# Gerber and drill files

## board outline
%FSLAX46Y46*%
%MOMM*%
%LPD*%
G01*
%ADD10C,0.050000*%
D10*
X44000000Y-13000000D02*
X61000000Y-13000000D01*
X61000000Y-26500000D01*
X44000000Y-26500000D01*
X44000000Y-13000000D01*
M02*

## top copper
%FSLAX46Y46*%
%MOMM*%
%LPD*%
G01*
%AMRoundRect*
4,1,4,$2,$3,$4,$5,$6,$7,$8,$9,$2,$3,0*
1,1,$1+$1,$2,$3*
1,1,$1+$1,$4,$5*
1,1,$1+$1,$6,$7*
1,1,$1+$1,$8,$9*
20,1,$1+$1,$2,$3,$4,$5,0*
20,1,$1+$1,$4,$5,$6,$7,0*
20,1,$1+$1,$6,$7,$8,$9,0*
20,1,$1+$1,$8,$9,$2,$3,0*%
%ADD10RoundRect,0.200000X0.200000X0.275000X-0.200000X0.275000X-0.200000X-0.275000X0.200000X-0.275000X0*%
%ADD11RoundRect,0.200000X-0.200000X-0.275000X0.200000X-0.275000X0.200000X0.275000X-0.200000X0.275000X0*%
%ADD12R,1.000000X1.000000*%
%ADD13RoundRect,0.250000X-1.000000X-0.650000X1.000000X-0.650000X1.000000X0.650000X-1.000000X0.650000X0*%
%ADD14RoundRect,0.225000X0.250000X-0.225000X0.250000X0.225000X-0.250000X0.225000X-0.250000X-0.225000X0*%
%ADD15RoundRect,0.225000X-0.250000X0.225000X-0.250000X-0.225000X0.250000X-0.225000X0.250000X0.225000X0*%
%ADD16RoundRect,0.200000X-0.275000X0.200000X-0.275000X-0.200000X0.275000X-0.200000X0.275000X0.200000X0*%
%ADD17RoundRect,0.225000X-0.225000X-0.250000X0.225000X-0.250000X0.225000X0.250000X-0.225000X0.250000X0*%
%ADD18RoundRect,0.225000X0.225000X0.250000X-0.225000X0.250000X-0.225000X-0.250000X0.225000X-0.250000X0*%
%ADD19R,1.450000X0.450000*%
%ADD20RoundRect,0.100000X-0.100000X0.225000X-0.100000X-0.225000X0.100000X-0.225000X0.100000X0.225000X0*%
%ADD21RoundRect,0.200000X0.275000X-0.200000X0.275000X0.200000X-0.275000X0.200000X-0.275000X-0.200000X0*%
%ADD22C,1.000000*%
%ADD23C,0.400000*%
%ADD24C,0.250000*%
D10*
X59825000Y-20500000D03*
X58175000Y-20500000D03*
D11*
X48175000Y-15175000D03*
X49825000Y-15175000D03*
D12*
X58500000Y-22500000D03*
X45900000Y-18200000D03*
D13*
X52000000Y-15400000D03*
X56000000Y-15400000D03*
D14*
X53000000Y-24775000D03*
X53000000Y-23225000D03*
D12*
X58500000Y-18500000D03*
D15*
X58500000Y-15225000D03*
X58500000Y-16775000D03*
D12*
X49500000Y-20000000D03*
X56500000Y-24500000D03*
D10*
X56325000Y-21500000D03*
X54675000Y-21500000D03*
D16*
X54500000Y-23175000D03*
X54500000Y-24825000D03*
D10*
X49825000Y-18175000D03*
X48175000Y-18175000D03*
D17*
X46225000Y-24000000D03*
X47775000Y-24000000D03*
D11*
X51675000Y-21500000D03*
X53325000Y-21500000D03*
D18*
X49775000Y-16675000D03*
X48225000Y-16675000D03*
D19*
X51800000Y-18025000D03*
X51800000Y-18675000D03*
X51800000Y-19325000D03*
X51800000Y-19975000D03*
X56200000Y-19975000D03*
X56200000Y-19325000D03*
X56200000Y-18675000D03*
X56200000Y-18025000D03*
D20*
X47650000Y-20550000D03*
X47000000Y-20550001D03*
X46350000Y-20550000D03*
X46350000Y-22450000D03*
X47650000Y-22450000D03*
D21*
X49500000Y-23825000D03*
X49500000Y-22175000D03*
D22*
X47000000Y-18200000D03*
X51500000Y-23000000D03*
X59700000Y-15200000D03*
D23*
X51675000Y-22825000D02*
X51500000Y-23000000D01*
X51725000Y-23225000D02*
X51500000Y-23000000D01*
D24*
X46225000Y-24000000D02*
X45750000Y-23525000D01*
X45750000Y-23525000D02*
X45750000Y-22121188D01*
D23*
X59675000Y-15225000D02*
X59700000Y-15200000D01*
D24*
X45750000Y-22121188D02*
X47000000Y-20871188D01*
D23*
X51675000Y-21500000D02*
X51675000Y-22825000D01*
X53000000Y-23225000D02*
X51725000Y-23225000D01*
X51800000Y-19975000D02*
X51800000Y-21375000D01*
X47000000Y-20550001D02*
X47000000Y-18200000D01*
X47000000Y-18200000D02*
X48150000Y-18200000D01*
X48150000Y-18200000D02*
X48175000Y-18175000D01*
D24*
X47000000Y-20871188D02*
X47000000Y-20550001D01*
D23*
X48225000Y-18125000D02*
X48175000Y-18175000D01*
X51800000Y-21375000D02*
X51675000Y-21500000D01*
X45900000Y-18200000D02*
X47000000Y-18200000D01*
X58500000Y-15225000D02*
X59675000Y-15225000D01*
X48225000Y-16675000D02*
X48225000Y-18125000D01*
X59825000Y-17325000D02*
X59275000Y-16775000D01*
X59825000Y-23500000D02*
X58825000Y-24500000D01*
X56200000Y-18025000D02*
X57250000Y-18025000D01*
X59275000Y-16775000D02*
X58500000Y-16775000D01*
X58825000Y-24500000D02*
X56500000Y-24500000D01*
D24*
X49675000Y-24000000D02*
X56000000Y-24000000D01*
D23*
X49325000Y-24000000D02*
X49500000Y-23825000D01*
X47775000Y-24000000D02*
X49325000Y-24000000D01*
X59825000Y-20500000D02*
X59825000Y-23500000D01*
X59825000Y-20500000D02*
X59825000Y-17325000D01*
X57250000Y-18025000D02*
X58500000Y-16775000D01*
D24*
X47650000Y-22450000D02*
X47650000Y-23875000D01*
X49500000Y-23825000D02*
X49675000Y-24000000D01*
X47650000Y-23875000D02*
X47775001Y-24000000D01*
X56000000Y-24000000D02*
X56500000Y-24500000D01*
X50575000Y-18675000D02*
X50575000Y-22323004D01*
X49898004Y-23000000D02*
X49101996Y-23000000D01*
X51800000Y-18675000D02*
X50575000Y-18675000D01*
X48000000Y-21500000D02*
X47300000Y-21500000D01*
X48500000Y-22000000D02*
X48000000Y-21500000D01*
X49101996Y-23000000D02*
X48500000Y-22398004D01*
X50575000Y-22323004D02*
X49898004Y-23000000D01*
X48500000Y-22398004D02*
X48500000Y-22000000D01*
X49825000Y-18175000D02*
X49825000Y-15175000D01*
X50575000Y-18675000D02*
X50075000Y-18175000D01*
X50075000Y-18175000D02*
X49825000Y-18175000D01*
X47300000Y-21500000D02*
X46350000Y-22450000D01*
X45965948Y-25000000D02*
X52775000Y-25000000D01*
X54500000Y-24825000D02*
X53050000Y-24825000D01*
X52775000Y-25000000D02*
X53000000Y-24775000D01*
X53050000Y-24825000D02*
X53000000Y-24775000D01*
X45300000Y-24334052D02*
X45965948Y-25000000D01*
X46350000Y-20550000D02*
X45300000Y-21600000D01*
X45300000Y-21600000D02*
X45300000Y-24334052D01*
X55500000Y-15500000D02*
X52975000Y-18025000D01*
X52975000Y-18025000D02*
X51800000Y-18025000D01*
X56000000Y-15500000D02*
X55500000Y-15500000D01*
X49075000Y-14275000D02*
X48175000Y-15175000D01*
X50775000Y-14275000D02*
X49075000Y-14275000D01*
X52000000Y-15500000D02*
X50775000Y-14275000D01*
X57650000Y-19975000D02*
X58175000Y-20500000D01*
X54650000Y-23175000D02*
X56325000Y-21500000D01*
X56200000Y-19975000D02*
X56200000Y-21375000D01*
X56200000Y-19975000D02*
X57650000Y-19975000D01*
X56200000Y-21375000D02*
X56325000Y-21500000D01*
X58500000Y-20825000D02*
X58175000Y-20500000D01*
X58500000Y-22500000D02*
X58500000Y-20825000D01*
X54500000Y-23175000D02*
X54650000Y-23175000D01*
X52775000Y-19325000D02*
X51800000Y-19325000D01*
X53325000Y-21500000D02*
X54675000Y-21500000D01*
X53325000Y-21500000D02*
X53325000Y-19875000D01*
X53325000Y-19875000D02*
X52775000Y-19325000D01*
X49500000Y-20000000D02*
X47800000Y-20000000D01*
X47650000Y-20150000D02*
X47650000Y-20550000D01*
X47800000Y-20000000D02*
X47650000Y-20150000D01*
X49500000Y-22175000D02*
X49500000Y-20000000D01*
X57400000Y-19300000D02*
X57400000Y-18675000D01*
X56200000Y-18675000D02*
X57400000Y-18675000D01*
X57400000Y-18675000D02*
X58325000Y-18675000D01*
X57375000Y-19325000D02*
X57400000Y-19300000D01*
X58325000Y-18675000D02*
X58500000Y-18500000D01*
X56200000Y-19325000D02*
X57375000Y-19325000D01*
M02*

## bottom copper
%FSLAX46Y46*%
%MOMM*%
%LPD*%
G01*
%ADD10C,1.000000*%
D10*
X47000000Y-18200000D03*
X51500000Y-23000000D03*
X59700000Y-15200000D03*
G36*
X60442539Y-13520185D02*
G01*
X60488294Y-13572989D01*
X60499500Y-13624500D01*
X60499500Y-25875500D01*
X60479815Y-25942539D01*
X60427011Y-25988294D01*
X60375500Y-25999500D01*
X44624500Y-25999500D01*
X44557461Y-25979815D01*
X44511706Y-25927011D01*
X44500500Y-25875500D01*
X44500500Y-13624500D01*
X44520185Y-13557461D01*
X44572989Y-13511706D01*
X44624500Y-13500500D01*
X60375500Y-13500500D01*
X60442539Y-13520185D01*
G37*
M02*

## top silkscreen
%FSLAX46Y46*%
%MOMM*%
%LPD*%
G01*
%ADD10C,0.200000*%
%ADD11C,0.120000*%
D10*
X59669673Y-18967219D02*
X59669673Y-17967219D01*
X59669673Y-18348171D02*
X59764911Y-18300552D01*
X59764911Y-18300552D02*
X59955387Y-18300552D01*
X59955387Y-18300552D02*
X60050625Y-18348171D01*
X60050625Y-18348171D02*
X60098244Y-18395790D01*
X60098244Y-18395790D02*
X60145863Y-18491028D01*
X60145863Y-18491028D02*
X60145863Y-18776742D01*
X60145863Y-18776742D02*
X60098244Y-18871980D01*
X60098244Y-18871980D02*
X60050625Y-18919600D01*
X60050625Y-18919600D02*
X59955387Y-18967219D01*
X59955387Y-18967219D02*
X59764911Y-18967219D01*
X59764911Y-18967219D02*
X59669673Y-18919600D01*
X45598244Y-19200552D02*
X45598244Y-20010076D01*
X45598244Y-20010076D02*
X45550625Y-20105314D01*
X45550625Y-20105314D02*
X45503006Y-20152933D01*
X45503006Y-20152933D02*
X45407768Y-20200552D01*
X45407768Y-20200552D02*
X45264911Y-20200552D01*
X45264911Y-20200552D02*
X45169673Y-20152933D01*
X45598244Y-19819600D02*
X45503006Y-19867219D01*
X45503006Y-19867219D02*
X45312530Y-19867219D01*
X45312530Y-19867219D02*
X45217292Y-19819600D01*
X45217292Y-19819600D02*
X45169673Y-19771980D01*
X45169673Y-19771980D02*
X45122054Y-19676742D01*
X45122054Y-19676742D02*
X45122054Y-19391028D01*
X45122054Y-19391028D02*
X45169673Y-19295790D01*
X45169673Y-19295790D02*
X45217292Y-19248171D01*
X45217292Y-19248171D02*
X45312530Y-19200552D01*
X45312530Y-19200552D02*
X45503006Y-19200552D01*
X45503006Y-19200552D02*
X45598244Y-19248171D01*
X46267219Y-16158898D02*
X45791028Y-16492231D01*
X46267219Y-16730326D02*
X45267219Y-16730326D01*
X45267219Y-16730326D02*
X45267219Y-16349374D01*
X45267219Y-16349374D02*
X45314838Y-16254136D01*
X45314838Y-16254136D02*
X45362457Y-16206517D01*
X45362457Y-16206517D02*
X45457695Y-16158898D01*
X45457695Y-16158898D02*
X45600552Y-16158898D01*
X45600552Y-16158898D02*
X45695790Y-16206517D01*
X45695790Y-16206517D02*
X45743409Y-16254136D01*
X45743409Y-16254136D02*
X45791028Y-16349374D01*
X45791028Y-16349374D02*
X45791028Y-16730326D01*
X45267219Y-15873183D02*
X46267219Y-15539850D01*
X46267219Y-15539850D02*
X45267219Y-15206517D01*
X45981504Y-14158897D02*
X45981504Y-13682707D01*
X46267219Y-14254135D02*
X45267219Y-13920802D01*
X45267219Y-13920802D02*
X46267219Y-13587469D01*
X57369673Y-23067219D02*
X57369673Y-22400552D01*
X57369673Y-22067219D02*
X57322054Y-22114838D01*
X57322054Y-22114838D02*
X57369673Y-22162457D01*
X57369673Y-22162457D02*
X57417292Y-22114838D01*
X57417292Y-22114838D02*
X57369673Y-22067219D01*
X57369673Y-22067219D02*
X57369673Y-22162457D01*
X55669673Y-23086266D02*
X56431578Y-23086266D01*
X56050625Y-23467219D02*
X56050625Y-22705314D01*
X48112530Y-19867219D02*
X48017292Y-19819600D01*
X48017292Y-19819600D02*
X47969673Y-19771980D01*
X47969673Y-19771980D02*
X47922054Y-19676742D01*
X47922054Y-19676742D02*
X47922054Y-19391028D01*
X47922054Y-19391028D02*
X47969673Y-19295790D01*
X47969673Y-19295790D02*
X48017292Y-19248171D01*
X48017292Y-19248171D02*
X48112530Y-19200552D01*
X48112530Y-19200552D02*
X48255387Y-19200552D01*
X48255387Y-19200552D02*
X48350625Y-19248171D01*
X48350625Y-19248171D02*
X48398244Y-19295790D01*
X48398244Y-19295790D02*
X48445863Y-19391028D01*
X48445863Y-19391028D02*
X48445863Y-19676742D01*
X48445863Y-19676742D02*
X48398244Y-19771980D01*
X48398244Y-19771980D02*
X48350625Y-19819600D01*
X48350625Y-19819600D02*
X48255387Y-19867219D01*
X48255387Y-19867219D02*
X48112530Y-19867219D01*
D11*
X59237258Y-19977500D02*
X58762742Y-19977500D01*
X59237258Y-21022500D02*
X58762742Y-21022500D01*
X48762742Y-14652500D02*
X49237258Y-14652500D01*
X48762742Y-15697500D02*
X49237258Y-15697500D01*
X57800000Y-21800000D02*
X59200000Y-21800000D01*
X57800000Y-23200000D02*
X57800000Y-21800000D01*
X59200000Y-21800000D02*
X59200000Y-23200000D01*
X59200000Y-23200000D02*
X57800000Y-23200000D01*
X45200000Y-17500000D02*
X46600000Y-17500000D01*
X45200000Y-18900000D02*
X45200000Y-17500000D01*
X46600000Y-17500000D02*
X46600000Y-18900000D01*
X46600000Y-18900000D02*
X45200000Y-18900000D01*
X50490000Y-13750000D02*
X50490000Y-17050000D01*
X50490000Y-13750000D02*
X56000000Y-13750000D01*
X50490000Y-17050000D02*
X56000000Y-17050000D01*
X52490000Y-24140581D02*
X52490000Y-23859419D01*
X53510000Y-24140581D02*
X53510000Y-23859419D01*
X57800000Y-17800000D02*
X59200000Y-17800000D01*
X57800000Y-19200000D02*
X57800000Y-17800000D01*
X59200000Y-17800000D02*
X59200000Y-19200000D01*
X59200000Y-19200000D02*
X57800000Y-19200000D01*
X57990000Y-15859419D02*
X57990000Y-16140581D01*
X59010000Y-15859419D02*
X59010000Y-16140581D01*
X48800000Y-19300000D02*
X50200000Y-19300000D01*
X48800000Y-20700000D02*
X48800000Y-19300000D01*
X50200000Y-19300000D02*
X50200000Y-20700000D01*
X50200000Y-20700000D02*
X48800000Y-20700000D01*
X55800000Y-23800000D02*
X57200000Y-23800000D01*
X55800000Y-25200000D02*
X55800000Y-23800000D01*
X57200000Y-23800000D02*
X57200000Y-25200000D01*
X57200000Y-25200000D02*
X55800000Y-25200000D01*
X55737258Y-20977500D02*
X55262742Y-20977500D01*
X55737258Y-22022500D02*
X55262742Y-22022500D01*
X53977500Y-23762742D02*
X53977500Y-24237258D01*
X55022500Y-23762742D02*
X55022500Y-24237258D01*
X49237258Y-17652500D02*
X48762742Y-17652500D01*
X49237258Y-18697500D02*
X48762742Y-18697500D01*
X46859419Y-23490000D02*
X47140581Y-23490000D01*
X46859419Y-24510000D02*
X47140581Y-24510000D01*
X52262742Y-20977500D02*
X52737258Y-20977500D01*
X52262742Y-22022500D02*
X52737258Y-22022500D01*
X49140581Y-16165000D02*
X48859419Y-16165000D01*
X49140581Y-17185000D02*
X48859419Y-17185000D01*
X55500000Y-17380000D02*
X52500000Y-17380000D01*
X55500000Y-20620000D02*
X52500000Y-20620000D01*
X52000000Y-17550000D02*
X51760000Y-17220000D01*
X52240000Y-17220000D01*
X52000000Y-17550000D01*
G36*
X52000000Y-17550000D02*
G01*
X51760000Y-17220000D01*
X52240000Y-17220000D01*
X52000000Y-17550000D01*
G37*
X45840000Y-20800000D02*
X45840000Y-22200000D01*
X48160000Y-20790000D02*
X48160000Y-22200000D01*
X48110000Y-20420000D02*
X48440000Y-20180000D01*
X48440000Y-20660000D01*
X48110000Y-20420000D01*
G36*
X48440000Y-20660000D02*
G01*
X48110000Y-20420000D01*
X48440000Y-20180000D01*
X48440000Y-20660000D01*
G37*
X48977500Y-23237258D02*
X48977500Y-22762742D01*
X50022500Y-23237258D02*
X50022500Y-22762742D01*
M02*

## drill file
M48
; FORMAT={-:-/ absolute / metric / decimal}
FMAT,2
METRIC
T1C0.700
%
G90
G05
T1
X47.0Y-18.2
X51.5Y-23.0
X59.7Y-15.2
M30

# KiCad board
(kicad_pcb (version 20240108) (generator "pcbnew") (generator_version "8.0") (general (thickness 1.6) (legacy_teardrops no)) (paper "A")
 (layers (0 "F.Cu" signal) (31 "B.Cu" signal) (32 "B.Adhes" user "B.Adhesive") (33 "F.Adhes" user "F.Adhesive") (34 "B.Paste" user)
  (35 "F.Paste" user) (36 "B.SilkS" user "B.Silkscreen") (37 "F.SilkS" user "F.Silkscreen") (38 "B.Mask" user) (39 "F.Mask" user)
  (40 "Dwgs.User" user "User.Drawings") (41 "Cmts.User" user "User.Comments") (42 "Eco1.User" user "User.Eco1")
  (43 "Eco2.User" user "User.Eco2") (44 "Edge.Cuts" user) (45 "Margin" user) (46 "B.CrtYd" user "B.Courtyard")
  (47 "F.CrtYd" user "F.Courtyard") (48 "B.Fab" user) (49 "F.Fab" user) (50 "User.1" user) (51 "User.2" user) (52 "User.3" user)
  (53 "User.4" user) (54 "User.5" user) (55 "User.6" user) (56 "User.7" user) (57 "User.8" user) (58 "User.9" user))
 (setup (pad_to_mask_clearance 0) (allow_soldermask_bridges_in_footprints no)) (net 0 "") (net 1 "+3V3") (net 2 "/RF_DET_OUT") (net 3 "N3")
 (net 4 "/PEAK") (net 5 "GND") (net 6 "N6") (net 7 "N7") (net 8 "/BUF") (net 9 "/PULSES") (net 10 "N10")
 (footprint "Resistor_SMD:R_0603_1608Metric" (layer "F.Cu") (at 59 20.5 180)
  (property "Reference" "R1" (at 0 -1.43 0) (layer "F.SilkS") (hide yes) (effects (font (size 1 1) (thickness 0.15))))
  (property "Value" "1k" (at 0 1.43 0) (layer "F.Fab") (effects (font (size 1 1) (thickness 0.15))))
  (fp_line (start -0.237258 0.5225) (end 0.237258 0.5225) (stroke (width 0.12) (type solid)) (layer "F.SilkS"))
  (fp_line (start -0.237258 -0.5225) (end 0.237258 -0.5225) (stroke (width 0.12) (type solid)) (layer "F.SilkS"))
  (pad "1" smd roundrect (at -0.825 0 180) (size 0.8 0.95) (layers "F.Cu" "F.Paste" "F.Mask") (roundrect_rratio 0.25) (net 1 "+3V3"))
  (pad "2" smd roundrect (at 0.825 0 180) (size 0.8 0.95) (layers "F.Cu" "F.Paste" "F.Mask") (roundrect_rratio 0.25) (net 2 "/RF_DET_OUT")))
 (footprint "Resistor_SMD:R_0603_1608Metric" (layer "F.Cu") (at 49 15.175)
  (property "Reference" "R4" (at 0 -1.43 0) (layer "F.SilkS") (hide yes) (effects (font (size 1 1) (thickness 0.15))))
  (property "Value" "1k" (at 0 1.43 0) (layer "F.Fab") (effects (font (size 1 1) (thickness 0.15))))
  (fp_line (start -0.237258 -0.5225) (end 0.237258 -0.5225) (stroke (width 0.12) (type solid)) (layer "F.SilkS"))
  (fp_line (start -0.237258 0.5225) (end 0.237258 0.5225) (stroke (width 0.12) (type solid)) (layer "F.SilkS"))
  (pad "1" smd roundrect (at -0.825 0) (size 0.8 0.95) (layers "F.Cu" "F.Paste" "F.Mask") (roundrect_rratio 0.25) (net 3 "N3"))
  (pad "2" smd roundrect (at 0.825 0) (size 0.8 0.95) (layers "F.Cu" "F.Paste" "F.Mask") (roundrect_rratio 0.25) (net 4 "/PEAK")))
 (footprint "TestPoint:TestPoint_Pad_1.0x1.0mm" (layer "F.Cu") (at 58.5 22.5)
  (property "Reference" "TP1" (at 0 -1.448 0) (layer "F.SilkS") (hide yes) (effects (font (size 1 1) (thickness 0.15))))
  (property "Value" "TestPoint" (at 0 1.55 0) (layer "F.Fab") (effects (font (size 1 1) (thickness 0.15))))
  (fp_line (start -0.7 -0.7) (end 0.7 -0.7) (stroke (width 0.12) (type solid)) (layer "F.SilkS"))
  (fp_line (start -0.7 0.7) (end -0.7 -0.7) (stroke (width 0.12) (type solid)) (layer "F.SilkS"))
  (fp_line (start 0.7 -0.7) (end 0.7 0.7) (stroke (width 0.12) (type solid)) (layer "F.SilkS"))
  (fp_line (start 0.7 0.7) (end -0.7 0.7) (stroke (width 0.12) (type solid)) (layer "F.SilkS"))
  (pad "1" smd rect (at 0 0) (size 1 1) (layers "F.Cu" "F.Mask") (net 2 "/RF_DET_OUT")))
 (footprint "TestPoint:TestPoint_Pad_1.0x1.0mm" (layer "F.Cu") (at 45.9 18.2 90)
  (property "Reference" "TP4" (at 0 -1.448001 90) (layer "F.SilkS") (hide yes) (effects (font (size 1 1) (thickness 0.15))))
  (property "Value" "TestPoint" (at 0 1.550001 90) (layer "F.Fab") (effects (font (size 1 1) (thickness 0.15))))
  (fp_line (start 0.7 -0.7) (end 0.7 0.7) (stroke (width 0.12) (type solid)) (layer "F.SilkS"))
  (fp_line (start -0.7 -0.7) (end 0.7 -0.7) (stroke (width 0.12) (type solid)) (layer "F.SilkS"))
  (fp_line (start 0.7 0.7) (end -0.7 0.7) (stroke (width 0.12) (type solid)) (layer "F.SilkS"))
  (fp_line (start -0.7 0.7) (end -0.7 -0.7) (stroke (width 0.12) (type solid)) (layer "F.SilkS"))
  (pad "1" smd rect (at 0 0 90) (size 1 1) (layers "F.Cu" "F.Mask") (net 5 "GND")))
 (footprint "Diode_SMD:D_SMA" (layer "F.Cu") (at 54 15.4)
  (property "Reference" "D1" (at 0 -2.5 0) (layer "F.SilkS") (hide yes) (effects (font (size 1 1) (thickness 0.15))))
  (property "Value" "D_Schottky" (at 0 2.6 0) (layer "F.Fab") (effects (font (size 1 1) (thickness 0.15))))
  (fp_line (start -3.51 -1.65) (end -3.51 1.65) (stroke (width 0.12) (type solid)) (layer "F.SilkS"))
  (fp_line (start -3.51 -1.65) (end 2 -1.65) (stroke (width 0.12) (type solid)) (layer "F.SilkS"))
  (fp_line (start -3.51 1.65) (end 2 1.65) (stroke (width 0.12) (type solid)) (layer "F.SilkS"))
  (pad "1" smd roundrect (at -2 0) (size 2.5 1.8) (layers "F.Cu" "F.Paste" "F.Mask") (roundrect_rratio 0.1388888889) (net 3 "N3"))
  (pad "2" smd roundrect (at 2 0) (size 2.5 1.8) (layers "F.Cu" "F.Paste" "F.Mask") (roundrect_rratio 0.1388888889) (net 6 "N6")))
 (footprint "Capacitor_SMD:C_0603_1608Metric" (layer "F.Cu") (at 53 24 90)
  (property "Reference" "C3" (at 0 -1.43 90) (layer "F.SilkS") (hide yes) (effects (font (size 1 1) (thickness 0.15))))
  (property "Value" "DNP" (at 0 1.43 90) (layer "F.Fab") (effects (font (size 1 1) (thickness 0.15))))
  (fp_line (start -0.140581 -0.51) (end 0.140581 -0.51) (stroke (width 0.12) (type solid)) (layer "F.SilkS"))
  (fp_line (start -0.140581 0.51) (end 0.140581 0.51) (stroke (width 0.12) (type solid)) (layer "F.SilkS"))
  (pad "1" smd roundrect (at -0.775 0 90) (size 0.9 0.95) (layers "F.Cu" "F.Paste" "F.Mask") (roundrect_rratio 0.25) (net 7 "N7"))
  (pad "2" smd roundrect (at 0.775 0 90) (size 0.9 0.95) (layers "F.Cu" "F.Paste" "F.Mask") (roundrect_rratio 0.25) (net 5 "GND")))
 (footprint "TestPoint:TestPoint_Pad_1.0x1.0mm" (layer "F.Cu") (at 58.5 18.5)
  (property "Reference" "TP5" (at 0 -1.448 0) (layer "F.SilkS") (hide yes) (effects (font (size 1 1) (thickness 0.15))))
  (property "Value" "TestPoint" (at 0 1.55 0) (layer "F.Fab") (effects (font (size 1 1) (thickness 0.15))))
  (fp_line (start -0.7 -0.7) (end 0.7 -0.7) (stroke (width 0.12) (type solid)) (layer "F.SilkS"))
  (fp_line (start -0.7 0.7) (end -0.7 -0.7) (stroke (width 0.12) (type solid)) (layer "F.SilkS"))
  (fp_line (start 0.7 -0.7) (end 0.7 0.7) (stroke (width 0.12) (type solid)) (layer "F.SilkS"))
  (fp_line (start 0.7 0.7) (end -0.7 0.7) (stroke (width 0.12) (type solid)) (layer "F.SilkS"))
  (pad "1" smd rect (at 0 0) (size 1 1) (layers "F.Cu" "F.Mask") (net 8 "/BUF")))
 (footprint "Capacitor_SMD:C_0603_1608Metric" (layer "F.Cu") (at 58.5 16 -90)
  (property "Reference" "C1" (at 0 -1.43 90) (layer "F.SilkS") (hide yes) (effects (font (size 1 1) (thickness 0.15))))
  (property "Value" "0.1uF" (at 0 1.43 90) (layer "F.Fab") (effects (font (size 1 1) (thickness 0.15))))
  (fp_line (start -0.140581 0.51) (end 0.140581 0.51) (stroke (width 0.12) (type solid)) (layer "F.SilkS"))
  (fp_line (start -0.140581 -0.51) (end 0.140581 -0.51) (stroke (width 0.12) (type solid)) (layer "F.SilkS"))
  (pad "1" smd roundrect (at -0.775 0 270) (size 0.9 0.95) (layers "F.Cu" "F.Paste" "F.Mask") (roundrect_rratio 0.25) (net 5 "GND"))
  (pad "2" smd roundrect (at 0.775 0 270) (size 0.9 0.95) (layers "F.Cu" "F.Paste" "F.Mask") (roundrect_rratio 0.25) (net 1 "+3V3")))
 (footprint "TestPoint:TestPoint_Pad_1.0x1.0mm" (layer "F.Cu") (at 49.5 20)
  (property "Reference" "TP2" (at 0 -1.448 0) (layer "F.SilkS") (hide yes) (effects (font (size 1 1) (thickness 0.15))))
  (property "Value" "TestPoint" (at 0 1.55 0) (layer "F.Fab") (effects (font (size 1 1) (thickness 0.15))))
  (fp_line (start -0.7 -0.7) (end 0.7 -0.7) (stroke (width 0.12) (type solid)) (layer "F.SilkS"))
  (fp_line (start -0.7 0.7) (end -0.7 -0.7) (stroke (width 0.12) (type solid)) (layer "F.SilkS"))
  (fp_line (start 0.7 -0.7) (end 0.7 0.7) (stroke (width 0.12) (type solid)) (layer "F.SilkS"))
  (fp_line (start 0.7 0.7) (end -0.7 0.7) (stroke (width 0.12) (type solid)) (layer "F.SilkS"))
  (pad "1" smd rect (at 0 0) (size 1 1) (layers "F.Cu" "F.Mask") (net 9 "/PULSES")))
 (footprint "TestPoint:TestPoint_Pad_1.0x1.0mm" (layer "F.Cu") (at 56.5 24.5)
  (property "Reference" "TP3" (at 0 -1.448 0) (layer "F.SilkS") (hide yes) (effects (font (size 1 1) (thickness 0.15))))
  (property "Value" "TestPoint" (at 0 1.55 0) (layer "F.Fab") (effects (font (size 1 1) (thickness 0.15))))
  (fp_line (start -0.7 -0.7) (end 0.7 -0.7) (stroke (width 0.12) (type solid)) (layer "F.SilkS"))
  (fp_line (start -0.7 0.7) (end -0.7 -0.7) (stroke (width 0.12) (type solid)) (layer "F.SilkS"))
  (fp_line (start 0.7 -0.7) (end 0.7 0.7) (stroke (width 0.12) (type solid)) (layer "F.SilkS"))
  (fp_line (start 0.7 0.7) (end -0.7 0.7) (stroke (width 0.12) (type solid)) (layer "F.SilkS"))
  (pad "1" smd rect (at 0 0) (size 1 1) (layers "F.Cu" "F.Mask") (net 1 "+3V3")))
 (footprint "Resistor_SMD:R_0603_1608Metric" (layer "F.Cu") (at 55.5 21.5 180)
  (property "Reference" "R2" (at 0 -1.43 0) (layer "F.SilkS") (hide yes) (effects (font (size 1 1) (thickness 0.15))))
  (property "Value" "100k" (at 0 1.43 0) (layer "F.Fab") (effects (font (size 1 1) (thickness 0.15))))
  (fp_line (start -0.237258 0.5225) (end 0.237258 0.5225) (stroke (width 0.12) (type solid)) (layer "F.SilkS"))
  (fp_line (start -0.237258 -0.5225) (end 0.237258 -0.5225) (stroke (width 0.12) (type solid)) (layer "F.SilkS"))
  (pad "1" smd roundrect (at -0.825 0 180) (size 0.8 0.95) (layers "F.Cu" "F.Paste" "F.Mask") (roundrect_rratio 0.25) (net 2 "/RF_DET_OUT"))
  (pad "2" smd roundrect (at 0.825 0 180) (size 0.8 0.95) (layers "F.Cu" "F.Paste" "F.Mask") (roundrect_rratio 0.25) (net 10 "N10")))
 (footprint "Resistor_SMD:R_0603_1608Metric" (layer "F.Cu") (at 54.5 24 -90)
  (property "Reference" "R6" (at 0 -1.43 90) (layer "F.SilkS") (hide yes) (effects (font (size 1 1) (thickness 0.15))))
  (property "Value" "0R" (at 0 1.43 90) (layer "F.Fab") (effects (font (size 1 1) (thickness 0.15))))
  (fp_line (start -0.237258 0.5225) (end 0.237258 0.5225) (stroke (width 0.12) (type solid)) (layer "F.SilkS"))
  (fp_line (start -0.237258 -0.5225) (end 0.237258 -0.5225) (stroke (width 0.12) (type solid)) (layer "F.SilkS"))
  (pad "1" smd roundrect (at -0.825 0 270) (size 0.8 0.95) (layers "F.Cu" "F.Paste" "F.Mask") (roundrect_rratio 0.25) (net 2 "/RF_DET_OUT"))
  (pad "2" smd roundrect (at 0.825 0 270) (size 0.8 0.95) (layers "F.Cu" "F.Paste" "F.Mask") (roundrect_rratio 0.25) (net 7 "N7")))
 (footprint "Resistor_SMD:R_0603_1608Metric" (layer "F.Cu") (at 49 18.175 180)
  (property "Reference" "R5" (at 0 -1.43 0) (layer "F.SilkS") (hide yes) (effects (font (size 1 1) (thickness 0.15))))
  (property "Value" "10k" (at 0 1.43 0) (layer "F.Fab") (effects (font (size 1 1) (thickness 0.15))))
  (fp_line (start -0.237258 0.5225) (end 0.237258 0.5225) (stroke (width 0.12) (type solid)) (layer "F.SilkS"))
  (fp_line (start -0.237258 -0.5225) (end 0.237258 -0.5225) (stroke (width 0.12) (type solid)) (layer "F.SilkS"))
  (pad "1" smd roundrect (at -0.825 0 180) (size 0.8 0.95) (layers "F.Cu" "F.Paste" "F.Mask") (roundrect_rratio 0.25) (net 4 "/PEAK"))
  (pad "2" smd roundrect (at 0.825 0 180) (size 0.8 0.95) (layers "F.Cu" "F.Paste" "F.Mask") (roundrect_rratio 0.25) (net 5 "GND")))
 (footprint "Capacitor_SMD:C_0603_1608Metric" (layer "F.Cu") (at 47 24)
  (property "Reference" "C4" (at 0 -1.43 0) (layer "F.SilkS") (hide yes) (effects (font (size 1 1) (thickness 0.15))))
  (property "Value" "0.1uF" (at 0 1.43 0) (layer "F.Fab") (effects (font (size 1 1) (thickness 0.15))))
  (fp_line (start -0.140581 -0.51) (end 0.140581 -0.51) (stroke (width 0.12) (type solid)) (layer "F.SilkS"))
  (fp_line (start -0.140581 0.51) (end 0.140581 0.51) (stroke (width 0.12) (type solid)) (layer "F.SilkS"))
  (pad "1" smd roundrect (at -0.775 0) (size 0.9 0.95) (layers "F.Cu" "F.Paste" "F.Mask") (roundrect_rratio 0.25) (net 5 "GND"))
  (pad "2" smd roundrect (at 0.775 0) (size 0.9 0.95) (layers "F.Cu" "F.Paste" "F.Mask") (roundrect_rratio 0.25) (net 1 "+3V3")))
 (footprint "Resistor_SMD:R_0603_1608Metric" (layer "F.Cu") (at 52.5 21.5)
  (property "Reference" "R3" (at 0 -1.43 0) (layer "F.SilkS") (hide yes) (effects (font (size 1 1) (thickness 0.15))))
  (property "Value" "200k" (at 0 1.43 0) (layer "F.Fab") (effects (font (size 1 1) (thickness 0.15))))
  (fp_line (start -0.237258 -0.5225) (end 0.237258 -0.5225) (stroke (width 0.12) (type solid)) (layer "F.SilkS"))
  (fp_line (start -0.237258 0.5225) (end 0.237258 0.5225) (stroke (width 0.12) (type solid)) (layer "F.SilkS"))
  (pad "1" smd roundrect (at -0.825 0) (size 0.8 0.95) (layers "F.Cu" "F.Paste" "F.Mask") (roundrect_rratio 0.25) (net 5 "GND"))
  (pad "2" smd roundrect (at 0.825 0) (size 0.8 0.95) (layers "F.Cu" "F.Paste" "F.Mask") (roundrect_rratio 0.25) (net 10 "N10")))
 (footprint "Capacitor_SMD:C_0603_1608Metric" (layer "F.Cu") (at 49 16.675 180)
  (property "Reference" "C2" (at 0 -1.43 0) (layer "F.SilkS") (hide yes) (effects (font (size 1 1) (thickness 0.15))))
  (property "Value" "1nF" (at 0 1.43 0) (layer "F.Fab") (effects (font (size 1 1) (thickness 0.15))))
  (fp_line (start -0.140581 0.51) (end 0.140581 0.51) (stroke (width 0.12) (type solid)) (layer "F.SilkS"))
  (fp_line (start -0.140581 -0.51) (end 0.140581 -0.51) (stroke (width 0.12) (type solid)) (layer "F.SilkS"))
  (pad "1" smd roundrect (at -0.775 0 180) (size 0.9 0.95) (layers "F.Cu" "F.Paste" "F.Mask") (roundrect_rratio 0.25) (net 4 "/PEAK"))
  (pad "2" smd roundrect (at 0.775 0 180) (size 0.9 0.95) (layers "F.Cu" "F.Paste" "F.Mask") (roundrect_rratio 0.25) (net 5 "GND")))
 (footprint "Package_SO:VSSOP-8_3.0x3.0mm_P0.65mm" (layer "F.Cu") (at 54 19)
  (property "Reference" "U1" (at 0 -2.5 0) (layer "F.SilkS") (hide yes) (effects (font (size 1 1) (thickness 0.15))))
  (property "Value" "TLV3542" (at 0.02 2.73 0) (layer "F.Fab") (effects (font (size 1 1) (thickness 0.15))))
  (fp_line (start 1.5 -1.62) (end -1.5 -1.62) (stroke (width 0.12) (type solid)) (layer "F.SilkS"))
  (fp_line (start 1.5 1.62) (end -1.5 1.62) (stroke (width 0.12) (type solid)) (layer "F.SilkS"))
  (fp_poly
   (pts (xy -2 -1.45) (xy -2.24 -1.78) (xy -1.76 -1.78) (xy -2 -1.45)) (stroke (width 0.12) (type solid)) (fill solid) (layer "F.SilkS"))
  (pad "1" smd rect (at -2.2 -0.975 270) (size 0.45 1.45) (layers "F.Cu" "F.Paste" "F.Mask") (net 6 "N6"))
  (pad "2" smd rect (at -2.2 -0.325 270) (size 0.45 1.45) (layers "F.Cu" "F.Paste" "F.Mask") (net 4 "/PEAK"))
  (pad "3" smd rect (at -2.2 0.325 270) (size 0.45 1.45) (layers "F.Cu" "F.Paste" "F.Mask") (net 10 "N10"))
  (pad "4" smd rect (at -2.2 0.975 270) (size 0.45 1.45) (layers "F.Cu" "F.Paste" "F.Mask") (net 5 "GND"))
  (pad "5" smd rect (at 2.2 0.975 270) (size 0.45 1.45) (layers "F.Cu" "F.Paste" "F.Mask") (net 2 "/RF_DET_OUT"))
  (pad "6" smd rect (at 2.2 0.325 270) (size 0.45 1.45) (layers "F.Cu" "F.Paste" "F.Mask") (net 8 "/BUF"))
  (pad "7" smd rect (at 2.2 -0.325 270) (size 0.45 1.45) (layers "F.Cu" "F.Paste" "F.Mask") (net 8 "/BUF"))
  (pad "8" smd rect (at 2.2 -0.975 270) (size 0.45 1.45) (layers "F.Cu" "F.Paste" "F.Mask") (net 1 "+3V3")))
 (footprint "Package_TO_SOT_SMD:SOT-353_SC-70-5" (layer "F.Cu") (at 47 21.5 -90)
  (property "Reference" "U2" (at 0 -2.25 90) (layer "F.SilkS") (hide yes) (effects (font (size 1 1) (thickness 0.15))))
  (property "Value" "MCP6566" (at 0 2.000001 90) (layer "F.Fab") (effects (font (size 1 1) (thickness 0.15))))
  (fp_line (start -0.7 1.16) (end 0.7 1.16) (stroke (width 0.12) (type solid)) (layer "F.SilkS"))
  (fp_line (start -0.71 -1.16) (end 0.7 -1.16) (stroke (width 0.12) (type solid)) (layer "F.SilkS"))
  (fp_poly
   (pts (xy -1.08 -1.11) (xy -1.32 -1.44) (xy -0.84 -1.44) (xy -1.08 -1.11)) (stroke (width 0.12) (type solid)) (fill solid)
   (layer "F.SilkS"))
  (pad "1" smd roundrect (at -0.95 -0.65 270) (size 0.65 0.4) (layers "F.Cu" "F.Paste" "F.Mask") (roundrect_rratio 0.25) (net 9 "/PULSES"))
  (pad "2" smd roundrect (at -0.949999 0 270) (size 0.65 0.4) (layers "F.Cu" "F.Paste" "F.Mask") (roundrect_rratio 0.25) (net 5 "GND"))
  (pad "3" smd roundrect (at -0.95 0.65 270) (size 0.65 0.4) (layers "F.Cu" "F.Paste" "F.Mask") (roundrect_rratio 0.25) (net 7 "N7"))
  (pad "4" smd roundrect (at 0.95 0.65 270) (size 0.65 0.4) (layers "F.Cu" "F.Paste" "F.Mask") (roundrect_rratio 0.25) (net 4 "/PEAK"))
  (pad "5" smd roundrect (at 0.95 -0.65 270) (size 0.65 0.4) (layers "F.Cu" "F.Paste" "F.Mask") (roundrect_rratio 0.25) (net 1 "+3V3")))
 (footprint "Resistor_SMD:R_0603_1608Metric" (layer "F.Cu") (at 49.5 23 90)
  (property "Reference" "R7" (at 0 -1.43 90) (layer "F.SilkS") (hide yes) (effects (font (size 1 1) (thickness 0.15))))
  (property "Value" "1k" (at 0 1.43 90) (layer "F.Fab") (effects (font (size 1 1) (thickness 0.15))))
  (fp_line (start -0.237258 -0.5225) (end 0.237258 -0.5225) (stroke (width 0.12) (type solid)) (layer "F.SilkS"))
  (fp_line (start -0.237258 0.5225) (end 0.237258 0.5225) (stroke (width 0.12) (type solid)) (layer "F.SilkS"))
  (pad "1" smd roundrect (at -0.825 0 90) (size 0.8 0.95) (layers "F.Cu" "F.Paste" "F.Mask") (roundrect_rratio 0.25) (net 1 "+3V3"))
  (pad "2" smd roundrect (at 0.825 0 90) (size 0.8 0.95) (layers "F.Cu" "F.Paste" "F.Mask") (roundrect_rratio 0.25) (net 9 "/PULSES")))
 (gr_rect (start 44 13) (end 61 26.5) (stroke (width 0.05) (type default)) (fill none) (layer "Edge.Cuts"))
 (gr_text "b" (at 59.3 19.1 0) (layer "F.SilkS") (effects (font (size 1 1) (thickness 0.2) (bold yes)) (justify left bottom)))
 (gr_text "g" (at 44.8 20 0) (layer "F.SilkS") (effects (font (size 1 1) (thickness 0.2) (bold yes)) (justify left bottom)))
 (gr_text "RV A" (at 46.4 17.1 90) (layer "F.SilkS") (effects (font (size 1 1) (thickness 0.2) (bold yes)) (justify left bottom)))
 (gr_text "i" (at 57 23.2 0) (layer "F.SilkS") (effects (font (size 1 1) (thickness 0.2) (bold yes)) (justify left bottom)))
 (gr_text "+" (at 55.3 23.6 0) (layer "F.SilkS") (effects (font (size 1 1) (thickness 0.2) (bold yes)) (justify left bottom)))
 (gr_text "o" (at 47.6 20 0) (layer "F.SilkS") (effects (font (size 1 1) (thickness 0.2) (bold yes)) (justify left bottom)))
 (segment (start 51.675 22.825) (end 51.5 23) (width 0.4) (layer "F.Cu") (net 5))
 (segment (start 51.725 23.225) (end 51.5 23) (width 0.4) (layer "F.Cu") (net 5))
 (segment (start 46.225 24) (end 45.75 23.525) (width 0.25) (layer "F.Cu") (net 5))
 (segment (start 45.75 23.525) (end 45.75 22.121188) (width 0.25) (layer "F.Cu") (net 5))
 (segment (start 59.675 15.225) (end 59.7 15.2) (width 0.4) (layer "F.Cu") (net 5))
 (segment (start 45.75 22.121188) (end 47 20.871188) (width 0.25) (layer "F.Cu") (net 5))
 (segment (start 51.675 21.5) (end 51.675 22.825) (width 0.4) (layer "F.Cu") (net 5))
 (segment (start 53 23.225) (end 51.725 23.225) (width 0.4) (layer "F.Cu") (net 5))
 (segment (start 51.8 19.975) (end 51.8 21.375) (width 0.4) (layer "F.Cu") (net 5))
 (segment (start 47 20.550001) (end 47 18.2) (width 0.4) (layer "F.Cu") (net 5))
 (segment (start 47 18.2) (end 48.15 18.2) (width 0.4) (layer "F.Cu") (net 5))
 (segment (start 48.15 18.2) (end 48.175 18.175) (width 0.4) (layer "F.Cu") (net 5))
 (segment (start 47 20.871188) (end 47 20.550001) (width 0.25) (layer "F.Cu") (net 5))
 (segment (start 48.225 18.125) (end 48.175 18.175) (width 0.4) (layer "F.Cu") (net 5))
 (segment (start 51.8 21.375) (end 51.675 21.5) (width 0.4) (layer "F.Cu") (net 5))
 (segment (start 45.9 18.2) (end 47 18.2) (width 0.4) (layer "F.Cu") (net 5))
 (segment (start 58.5 15.225) (end 59.675 15.225) (width 0.4) (layer "F.Cu") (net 5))
 (segment (start 48.225 16.675) (end 48.225 18.125) (width 0.4) (layer "F.Cu") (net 5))
 (via (at 47 18.2) (size 1) (drill 0.7) (layers "F.Cu" "B.Cu") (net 5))
 (via (at 51.5 23) (size 1) (drill 0.7) (layers "F.Cu" "B.Cu") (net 5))
 (via (at 59.7 15.2) (size 1) (drill 0.7) (layers "F.Cu" "B.Cu") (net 5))
 (segment (start 59.825 17.325) (end 59.275 16.775) (width 0.4) (layer "F.Cu") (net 1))
 (segment (start 59.825 23.5) (end 58.825 24.5) (width 0.4) (layer "F.Cu") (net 1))
 (segment (start 56.2 18.025) (end 57.25 18.025) (width 0.4) (layer "F.Cu") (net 1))
 (segment (start 59.275 16.775) (end 58.5 16.775) (width 0.4) (layer "F.Cu") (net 1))
 (segment (start 58.825 24.5) (end 56.5 24.5) (width 0.4) (layer "F.Cu") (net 1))
 (segment (start 49.675 24) (end 56 24) (width 0.25) (layer "F.Cu") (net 1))
 (segment (start 49.325 24) (end 49.5 23.825) (width 0.4) (layer "F.Cu") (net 1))
 (segment (start 47.775 24) (end 49.325 24) (width 0.4) (layer "F.Cu") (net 1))
 (segment (start 59.825 20.5) (end 59.825 23.5) (width 0.4) (layer "F.Cu") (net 1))
 (segment (start 59.825 20.5) (end 59.825 17.325) (width 0.4) (layer "F.Cu") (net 1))
 (segment (start 57.25 18.025) (end 58.5 16.775) (width 0.4) (layer "F.Cu") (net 1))
 (segment (start 47.65 22.45) (end 47.65 23.875) (width 0.25) (layer "F.Cu") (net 1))
 (segment (start 49.5 23.825) (end 49.675 24) (width 0.25) (layer "F.Cu") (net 1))
 (segment (start 47.65 23.875) (end 47.775001 24) (width 0.25) (layer "F.Cu") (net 1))
 (segment (start 56 24) (end 56.5 24.5) (width 0.25) (layer "F.Cu") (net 1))
 (segment (start 50.575 18.675) (end 50.575 22.323004) (width 0.25) (layer "F.Cu") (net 4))
 (segment (start 49.898004 23) (end 49.101996 23) (width 0.25) (layer "F.Cu") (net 4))
 (segment (start 51.8 18.675) (end 50.575 18.675) (width 0.25) (layer "F.Cu") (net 4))
 (segment (start 48 21.5) (end 47.3 21.5) (width 0.25) (layer "F.Cu") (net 4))
 (segment (start 48.5 22) (end 48 21.5) (width 0.25) (layer "F.Cu") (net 4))
 (segment (start 49.101996 23) (end 48.5 22.398004) (width 0.25) (layer "F.Cu") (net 4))
 (segment (start 50.575 22.323004) (end 49.898004 23) (width 0.25) (layer "F.Cu") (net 4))
 (segment (start 48.5 22.398004) (end 48.5 22) (width 0.25) (layer "F.Cu") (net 4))
 (segment (start 49.825 18.175) (end 49.825 15.175) (width 0.25) (layer "F.Cu") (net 4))
 (segment (start 50.575 18.675) (end 50.075 18.175) (width 0.25) (layer "F.Cu") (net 4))
 (segment (start 50.075 18.175) (end 49.825 18.175) (width 0.25) (layer "F.Cu") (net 4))
 (segment (start 47.3 21.5) (end 46.35 22.45) (width 0.25) (layer "F.Cu") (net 4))
 (segment (start 45.965948 25) (end 52.775 25) (width 0.25) (layer "F.Cu") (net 7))
 (segment (start 54.5 24.825) (end 53.05 24.825) (width 0.25) (layer "F.Cu") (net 7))
 (segment (start 52.775 25) (end 53 24.775) (width 0.25) (layer "F.Cu") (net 7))
 (segment (start 53.05 24.825) (end 53 24.775) (width 0.25) (layer "F.Cu") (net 7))
 (segment (start 45.3 24.334052) (end 45.965948 25) (width 0.25) (layer "F.Cu") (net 7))
 (segment (start 46.35 20.55) (end 45.3 21.6) (width 0.25) (layer "F.Cu") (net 7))
 (segment (start 45.3 21.6) (end 45.3 24.334052) (width 0.25) (layer "F.Cu") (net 7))
 (segment (start 55.5 15.5) (end 52.975 18.025) (width 0.25) (layer "F.Cu") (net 6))
 (segment (start 52.975 18.025) (end 51.8 18.025) (width 0.25) (layer "F.Cu") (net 6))
 (segment (start 56 15.5) (end 55.5 15.5) (width 0.25) (layer "F.Cu") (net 6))
 (segment (start 49.075 14.275) (end 48.175 15.175) (width 0.25) (layer "F.Cu") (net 3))
 (segment (start 50.775 14.275) (end 49.075 14.275) (width 0.25) (layer "F.Cu") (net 3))
 (segment (start 52 15.5) (end 50.775 14.275) (width 0.25) (layer "F.Cu") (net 3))
 (segment (start 57.65 19.975) (end 58.175 20.5) (width 0.25) (layer "F.Cu") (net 2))
 (segment (start 54.65 23.175) (end 56.325 21.5) (width 0.25) (layer "F.Cu") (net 2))
 (segment (start 56.2 19.975) (end 56.2 21.375) (width 0.25) (layer "F.Cu") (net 2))
 (segment (start 56.2 19.975) (end 57.65 19.975) (width 0.25) (layer "F.Cu") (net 2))
 (segment (start 56.2 21.375) (end 56.325 21.5) (width 0.25) (layer "F.Cu") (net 2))
 (segment (start 58.5 20.825) (end 58.175 20.5) (width 0.25) (layer "F.Cu") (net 2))
 (segment (start 58.5 22.5) (end 58.5 20.825) (width 0.25) (layer "F.Cu") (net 2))
 (segment (start 54.5 23.175) (end 54.65 23.175) (width 0.25) (layer "F.Cu") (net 2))
 (segment (start 52.775 19.325) (end 51.8 19.325) (width 0.25) (layer "F.Cu") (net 10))
 (segment (start 53.325 21.5) (end 54.675 21.5) (width 0.25) (layer "F.Cu") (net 10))
 (segment (start 53.325 21.5) (end 53.325 19.875) (width 0.25) (layer "F.Cu") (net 10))
 (segment (start 53.325 19.875) (end 52.775 19.325) (width 0.25) (layer "F.Cu") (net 10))
 (segment (start 49.5 20) (end 47.8 20) (width 0.25) (layer "F.Cu") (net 9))
 (segment (start 47.65 20.15) (end 47.65 20.55) (width 0.25) (layer "F.Cu") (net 9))
 (segment (start 47.8 20) (end 47.65 20.15) (width 0.25) (layer "F.Cu") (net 9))
 (segment (start 49.5 22.175) (end 49.5 20) (width 0.25) (layer "F.Cu") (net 9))
 (segment (start 57.4 19.3) (end 57.4 18.675) (width 0.25) (layer "F.Cu") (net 8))
 (segment (start 56.2 18.675) (end 57.4 18.675) (width 0.25) (layer "F.Cu") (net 8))
 (segment (start 57.4 18.675) (end 58.325 18.675) (width 0.25) (layer "F.Cu") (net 8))
 (segment (start 57.375 19.325) (end 57.4 19.3) (width 0.25) (layer "F.Cu") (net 8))
 (segment (start 58.325 18.675) (end 58.5 18.5) (width 0.25) (layer "F.Cu") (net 8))
 (segment (start 56.2 19.325) (end 57.375 19.325) (width 0.25) (layer "F.Cu") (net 8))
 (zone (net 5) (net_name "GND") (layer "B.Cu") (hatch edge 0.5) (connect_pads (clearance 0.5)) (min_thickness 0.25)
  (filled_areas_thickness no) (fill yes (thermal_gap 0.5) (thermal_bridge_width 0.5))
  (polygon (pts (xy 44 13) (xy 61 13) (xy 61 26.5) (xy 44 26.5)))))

